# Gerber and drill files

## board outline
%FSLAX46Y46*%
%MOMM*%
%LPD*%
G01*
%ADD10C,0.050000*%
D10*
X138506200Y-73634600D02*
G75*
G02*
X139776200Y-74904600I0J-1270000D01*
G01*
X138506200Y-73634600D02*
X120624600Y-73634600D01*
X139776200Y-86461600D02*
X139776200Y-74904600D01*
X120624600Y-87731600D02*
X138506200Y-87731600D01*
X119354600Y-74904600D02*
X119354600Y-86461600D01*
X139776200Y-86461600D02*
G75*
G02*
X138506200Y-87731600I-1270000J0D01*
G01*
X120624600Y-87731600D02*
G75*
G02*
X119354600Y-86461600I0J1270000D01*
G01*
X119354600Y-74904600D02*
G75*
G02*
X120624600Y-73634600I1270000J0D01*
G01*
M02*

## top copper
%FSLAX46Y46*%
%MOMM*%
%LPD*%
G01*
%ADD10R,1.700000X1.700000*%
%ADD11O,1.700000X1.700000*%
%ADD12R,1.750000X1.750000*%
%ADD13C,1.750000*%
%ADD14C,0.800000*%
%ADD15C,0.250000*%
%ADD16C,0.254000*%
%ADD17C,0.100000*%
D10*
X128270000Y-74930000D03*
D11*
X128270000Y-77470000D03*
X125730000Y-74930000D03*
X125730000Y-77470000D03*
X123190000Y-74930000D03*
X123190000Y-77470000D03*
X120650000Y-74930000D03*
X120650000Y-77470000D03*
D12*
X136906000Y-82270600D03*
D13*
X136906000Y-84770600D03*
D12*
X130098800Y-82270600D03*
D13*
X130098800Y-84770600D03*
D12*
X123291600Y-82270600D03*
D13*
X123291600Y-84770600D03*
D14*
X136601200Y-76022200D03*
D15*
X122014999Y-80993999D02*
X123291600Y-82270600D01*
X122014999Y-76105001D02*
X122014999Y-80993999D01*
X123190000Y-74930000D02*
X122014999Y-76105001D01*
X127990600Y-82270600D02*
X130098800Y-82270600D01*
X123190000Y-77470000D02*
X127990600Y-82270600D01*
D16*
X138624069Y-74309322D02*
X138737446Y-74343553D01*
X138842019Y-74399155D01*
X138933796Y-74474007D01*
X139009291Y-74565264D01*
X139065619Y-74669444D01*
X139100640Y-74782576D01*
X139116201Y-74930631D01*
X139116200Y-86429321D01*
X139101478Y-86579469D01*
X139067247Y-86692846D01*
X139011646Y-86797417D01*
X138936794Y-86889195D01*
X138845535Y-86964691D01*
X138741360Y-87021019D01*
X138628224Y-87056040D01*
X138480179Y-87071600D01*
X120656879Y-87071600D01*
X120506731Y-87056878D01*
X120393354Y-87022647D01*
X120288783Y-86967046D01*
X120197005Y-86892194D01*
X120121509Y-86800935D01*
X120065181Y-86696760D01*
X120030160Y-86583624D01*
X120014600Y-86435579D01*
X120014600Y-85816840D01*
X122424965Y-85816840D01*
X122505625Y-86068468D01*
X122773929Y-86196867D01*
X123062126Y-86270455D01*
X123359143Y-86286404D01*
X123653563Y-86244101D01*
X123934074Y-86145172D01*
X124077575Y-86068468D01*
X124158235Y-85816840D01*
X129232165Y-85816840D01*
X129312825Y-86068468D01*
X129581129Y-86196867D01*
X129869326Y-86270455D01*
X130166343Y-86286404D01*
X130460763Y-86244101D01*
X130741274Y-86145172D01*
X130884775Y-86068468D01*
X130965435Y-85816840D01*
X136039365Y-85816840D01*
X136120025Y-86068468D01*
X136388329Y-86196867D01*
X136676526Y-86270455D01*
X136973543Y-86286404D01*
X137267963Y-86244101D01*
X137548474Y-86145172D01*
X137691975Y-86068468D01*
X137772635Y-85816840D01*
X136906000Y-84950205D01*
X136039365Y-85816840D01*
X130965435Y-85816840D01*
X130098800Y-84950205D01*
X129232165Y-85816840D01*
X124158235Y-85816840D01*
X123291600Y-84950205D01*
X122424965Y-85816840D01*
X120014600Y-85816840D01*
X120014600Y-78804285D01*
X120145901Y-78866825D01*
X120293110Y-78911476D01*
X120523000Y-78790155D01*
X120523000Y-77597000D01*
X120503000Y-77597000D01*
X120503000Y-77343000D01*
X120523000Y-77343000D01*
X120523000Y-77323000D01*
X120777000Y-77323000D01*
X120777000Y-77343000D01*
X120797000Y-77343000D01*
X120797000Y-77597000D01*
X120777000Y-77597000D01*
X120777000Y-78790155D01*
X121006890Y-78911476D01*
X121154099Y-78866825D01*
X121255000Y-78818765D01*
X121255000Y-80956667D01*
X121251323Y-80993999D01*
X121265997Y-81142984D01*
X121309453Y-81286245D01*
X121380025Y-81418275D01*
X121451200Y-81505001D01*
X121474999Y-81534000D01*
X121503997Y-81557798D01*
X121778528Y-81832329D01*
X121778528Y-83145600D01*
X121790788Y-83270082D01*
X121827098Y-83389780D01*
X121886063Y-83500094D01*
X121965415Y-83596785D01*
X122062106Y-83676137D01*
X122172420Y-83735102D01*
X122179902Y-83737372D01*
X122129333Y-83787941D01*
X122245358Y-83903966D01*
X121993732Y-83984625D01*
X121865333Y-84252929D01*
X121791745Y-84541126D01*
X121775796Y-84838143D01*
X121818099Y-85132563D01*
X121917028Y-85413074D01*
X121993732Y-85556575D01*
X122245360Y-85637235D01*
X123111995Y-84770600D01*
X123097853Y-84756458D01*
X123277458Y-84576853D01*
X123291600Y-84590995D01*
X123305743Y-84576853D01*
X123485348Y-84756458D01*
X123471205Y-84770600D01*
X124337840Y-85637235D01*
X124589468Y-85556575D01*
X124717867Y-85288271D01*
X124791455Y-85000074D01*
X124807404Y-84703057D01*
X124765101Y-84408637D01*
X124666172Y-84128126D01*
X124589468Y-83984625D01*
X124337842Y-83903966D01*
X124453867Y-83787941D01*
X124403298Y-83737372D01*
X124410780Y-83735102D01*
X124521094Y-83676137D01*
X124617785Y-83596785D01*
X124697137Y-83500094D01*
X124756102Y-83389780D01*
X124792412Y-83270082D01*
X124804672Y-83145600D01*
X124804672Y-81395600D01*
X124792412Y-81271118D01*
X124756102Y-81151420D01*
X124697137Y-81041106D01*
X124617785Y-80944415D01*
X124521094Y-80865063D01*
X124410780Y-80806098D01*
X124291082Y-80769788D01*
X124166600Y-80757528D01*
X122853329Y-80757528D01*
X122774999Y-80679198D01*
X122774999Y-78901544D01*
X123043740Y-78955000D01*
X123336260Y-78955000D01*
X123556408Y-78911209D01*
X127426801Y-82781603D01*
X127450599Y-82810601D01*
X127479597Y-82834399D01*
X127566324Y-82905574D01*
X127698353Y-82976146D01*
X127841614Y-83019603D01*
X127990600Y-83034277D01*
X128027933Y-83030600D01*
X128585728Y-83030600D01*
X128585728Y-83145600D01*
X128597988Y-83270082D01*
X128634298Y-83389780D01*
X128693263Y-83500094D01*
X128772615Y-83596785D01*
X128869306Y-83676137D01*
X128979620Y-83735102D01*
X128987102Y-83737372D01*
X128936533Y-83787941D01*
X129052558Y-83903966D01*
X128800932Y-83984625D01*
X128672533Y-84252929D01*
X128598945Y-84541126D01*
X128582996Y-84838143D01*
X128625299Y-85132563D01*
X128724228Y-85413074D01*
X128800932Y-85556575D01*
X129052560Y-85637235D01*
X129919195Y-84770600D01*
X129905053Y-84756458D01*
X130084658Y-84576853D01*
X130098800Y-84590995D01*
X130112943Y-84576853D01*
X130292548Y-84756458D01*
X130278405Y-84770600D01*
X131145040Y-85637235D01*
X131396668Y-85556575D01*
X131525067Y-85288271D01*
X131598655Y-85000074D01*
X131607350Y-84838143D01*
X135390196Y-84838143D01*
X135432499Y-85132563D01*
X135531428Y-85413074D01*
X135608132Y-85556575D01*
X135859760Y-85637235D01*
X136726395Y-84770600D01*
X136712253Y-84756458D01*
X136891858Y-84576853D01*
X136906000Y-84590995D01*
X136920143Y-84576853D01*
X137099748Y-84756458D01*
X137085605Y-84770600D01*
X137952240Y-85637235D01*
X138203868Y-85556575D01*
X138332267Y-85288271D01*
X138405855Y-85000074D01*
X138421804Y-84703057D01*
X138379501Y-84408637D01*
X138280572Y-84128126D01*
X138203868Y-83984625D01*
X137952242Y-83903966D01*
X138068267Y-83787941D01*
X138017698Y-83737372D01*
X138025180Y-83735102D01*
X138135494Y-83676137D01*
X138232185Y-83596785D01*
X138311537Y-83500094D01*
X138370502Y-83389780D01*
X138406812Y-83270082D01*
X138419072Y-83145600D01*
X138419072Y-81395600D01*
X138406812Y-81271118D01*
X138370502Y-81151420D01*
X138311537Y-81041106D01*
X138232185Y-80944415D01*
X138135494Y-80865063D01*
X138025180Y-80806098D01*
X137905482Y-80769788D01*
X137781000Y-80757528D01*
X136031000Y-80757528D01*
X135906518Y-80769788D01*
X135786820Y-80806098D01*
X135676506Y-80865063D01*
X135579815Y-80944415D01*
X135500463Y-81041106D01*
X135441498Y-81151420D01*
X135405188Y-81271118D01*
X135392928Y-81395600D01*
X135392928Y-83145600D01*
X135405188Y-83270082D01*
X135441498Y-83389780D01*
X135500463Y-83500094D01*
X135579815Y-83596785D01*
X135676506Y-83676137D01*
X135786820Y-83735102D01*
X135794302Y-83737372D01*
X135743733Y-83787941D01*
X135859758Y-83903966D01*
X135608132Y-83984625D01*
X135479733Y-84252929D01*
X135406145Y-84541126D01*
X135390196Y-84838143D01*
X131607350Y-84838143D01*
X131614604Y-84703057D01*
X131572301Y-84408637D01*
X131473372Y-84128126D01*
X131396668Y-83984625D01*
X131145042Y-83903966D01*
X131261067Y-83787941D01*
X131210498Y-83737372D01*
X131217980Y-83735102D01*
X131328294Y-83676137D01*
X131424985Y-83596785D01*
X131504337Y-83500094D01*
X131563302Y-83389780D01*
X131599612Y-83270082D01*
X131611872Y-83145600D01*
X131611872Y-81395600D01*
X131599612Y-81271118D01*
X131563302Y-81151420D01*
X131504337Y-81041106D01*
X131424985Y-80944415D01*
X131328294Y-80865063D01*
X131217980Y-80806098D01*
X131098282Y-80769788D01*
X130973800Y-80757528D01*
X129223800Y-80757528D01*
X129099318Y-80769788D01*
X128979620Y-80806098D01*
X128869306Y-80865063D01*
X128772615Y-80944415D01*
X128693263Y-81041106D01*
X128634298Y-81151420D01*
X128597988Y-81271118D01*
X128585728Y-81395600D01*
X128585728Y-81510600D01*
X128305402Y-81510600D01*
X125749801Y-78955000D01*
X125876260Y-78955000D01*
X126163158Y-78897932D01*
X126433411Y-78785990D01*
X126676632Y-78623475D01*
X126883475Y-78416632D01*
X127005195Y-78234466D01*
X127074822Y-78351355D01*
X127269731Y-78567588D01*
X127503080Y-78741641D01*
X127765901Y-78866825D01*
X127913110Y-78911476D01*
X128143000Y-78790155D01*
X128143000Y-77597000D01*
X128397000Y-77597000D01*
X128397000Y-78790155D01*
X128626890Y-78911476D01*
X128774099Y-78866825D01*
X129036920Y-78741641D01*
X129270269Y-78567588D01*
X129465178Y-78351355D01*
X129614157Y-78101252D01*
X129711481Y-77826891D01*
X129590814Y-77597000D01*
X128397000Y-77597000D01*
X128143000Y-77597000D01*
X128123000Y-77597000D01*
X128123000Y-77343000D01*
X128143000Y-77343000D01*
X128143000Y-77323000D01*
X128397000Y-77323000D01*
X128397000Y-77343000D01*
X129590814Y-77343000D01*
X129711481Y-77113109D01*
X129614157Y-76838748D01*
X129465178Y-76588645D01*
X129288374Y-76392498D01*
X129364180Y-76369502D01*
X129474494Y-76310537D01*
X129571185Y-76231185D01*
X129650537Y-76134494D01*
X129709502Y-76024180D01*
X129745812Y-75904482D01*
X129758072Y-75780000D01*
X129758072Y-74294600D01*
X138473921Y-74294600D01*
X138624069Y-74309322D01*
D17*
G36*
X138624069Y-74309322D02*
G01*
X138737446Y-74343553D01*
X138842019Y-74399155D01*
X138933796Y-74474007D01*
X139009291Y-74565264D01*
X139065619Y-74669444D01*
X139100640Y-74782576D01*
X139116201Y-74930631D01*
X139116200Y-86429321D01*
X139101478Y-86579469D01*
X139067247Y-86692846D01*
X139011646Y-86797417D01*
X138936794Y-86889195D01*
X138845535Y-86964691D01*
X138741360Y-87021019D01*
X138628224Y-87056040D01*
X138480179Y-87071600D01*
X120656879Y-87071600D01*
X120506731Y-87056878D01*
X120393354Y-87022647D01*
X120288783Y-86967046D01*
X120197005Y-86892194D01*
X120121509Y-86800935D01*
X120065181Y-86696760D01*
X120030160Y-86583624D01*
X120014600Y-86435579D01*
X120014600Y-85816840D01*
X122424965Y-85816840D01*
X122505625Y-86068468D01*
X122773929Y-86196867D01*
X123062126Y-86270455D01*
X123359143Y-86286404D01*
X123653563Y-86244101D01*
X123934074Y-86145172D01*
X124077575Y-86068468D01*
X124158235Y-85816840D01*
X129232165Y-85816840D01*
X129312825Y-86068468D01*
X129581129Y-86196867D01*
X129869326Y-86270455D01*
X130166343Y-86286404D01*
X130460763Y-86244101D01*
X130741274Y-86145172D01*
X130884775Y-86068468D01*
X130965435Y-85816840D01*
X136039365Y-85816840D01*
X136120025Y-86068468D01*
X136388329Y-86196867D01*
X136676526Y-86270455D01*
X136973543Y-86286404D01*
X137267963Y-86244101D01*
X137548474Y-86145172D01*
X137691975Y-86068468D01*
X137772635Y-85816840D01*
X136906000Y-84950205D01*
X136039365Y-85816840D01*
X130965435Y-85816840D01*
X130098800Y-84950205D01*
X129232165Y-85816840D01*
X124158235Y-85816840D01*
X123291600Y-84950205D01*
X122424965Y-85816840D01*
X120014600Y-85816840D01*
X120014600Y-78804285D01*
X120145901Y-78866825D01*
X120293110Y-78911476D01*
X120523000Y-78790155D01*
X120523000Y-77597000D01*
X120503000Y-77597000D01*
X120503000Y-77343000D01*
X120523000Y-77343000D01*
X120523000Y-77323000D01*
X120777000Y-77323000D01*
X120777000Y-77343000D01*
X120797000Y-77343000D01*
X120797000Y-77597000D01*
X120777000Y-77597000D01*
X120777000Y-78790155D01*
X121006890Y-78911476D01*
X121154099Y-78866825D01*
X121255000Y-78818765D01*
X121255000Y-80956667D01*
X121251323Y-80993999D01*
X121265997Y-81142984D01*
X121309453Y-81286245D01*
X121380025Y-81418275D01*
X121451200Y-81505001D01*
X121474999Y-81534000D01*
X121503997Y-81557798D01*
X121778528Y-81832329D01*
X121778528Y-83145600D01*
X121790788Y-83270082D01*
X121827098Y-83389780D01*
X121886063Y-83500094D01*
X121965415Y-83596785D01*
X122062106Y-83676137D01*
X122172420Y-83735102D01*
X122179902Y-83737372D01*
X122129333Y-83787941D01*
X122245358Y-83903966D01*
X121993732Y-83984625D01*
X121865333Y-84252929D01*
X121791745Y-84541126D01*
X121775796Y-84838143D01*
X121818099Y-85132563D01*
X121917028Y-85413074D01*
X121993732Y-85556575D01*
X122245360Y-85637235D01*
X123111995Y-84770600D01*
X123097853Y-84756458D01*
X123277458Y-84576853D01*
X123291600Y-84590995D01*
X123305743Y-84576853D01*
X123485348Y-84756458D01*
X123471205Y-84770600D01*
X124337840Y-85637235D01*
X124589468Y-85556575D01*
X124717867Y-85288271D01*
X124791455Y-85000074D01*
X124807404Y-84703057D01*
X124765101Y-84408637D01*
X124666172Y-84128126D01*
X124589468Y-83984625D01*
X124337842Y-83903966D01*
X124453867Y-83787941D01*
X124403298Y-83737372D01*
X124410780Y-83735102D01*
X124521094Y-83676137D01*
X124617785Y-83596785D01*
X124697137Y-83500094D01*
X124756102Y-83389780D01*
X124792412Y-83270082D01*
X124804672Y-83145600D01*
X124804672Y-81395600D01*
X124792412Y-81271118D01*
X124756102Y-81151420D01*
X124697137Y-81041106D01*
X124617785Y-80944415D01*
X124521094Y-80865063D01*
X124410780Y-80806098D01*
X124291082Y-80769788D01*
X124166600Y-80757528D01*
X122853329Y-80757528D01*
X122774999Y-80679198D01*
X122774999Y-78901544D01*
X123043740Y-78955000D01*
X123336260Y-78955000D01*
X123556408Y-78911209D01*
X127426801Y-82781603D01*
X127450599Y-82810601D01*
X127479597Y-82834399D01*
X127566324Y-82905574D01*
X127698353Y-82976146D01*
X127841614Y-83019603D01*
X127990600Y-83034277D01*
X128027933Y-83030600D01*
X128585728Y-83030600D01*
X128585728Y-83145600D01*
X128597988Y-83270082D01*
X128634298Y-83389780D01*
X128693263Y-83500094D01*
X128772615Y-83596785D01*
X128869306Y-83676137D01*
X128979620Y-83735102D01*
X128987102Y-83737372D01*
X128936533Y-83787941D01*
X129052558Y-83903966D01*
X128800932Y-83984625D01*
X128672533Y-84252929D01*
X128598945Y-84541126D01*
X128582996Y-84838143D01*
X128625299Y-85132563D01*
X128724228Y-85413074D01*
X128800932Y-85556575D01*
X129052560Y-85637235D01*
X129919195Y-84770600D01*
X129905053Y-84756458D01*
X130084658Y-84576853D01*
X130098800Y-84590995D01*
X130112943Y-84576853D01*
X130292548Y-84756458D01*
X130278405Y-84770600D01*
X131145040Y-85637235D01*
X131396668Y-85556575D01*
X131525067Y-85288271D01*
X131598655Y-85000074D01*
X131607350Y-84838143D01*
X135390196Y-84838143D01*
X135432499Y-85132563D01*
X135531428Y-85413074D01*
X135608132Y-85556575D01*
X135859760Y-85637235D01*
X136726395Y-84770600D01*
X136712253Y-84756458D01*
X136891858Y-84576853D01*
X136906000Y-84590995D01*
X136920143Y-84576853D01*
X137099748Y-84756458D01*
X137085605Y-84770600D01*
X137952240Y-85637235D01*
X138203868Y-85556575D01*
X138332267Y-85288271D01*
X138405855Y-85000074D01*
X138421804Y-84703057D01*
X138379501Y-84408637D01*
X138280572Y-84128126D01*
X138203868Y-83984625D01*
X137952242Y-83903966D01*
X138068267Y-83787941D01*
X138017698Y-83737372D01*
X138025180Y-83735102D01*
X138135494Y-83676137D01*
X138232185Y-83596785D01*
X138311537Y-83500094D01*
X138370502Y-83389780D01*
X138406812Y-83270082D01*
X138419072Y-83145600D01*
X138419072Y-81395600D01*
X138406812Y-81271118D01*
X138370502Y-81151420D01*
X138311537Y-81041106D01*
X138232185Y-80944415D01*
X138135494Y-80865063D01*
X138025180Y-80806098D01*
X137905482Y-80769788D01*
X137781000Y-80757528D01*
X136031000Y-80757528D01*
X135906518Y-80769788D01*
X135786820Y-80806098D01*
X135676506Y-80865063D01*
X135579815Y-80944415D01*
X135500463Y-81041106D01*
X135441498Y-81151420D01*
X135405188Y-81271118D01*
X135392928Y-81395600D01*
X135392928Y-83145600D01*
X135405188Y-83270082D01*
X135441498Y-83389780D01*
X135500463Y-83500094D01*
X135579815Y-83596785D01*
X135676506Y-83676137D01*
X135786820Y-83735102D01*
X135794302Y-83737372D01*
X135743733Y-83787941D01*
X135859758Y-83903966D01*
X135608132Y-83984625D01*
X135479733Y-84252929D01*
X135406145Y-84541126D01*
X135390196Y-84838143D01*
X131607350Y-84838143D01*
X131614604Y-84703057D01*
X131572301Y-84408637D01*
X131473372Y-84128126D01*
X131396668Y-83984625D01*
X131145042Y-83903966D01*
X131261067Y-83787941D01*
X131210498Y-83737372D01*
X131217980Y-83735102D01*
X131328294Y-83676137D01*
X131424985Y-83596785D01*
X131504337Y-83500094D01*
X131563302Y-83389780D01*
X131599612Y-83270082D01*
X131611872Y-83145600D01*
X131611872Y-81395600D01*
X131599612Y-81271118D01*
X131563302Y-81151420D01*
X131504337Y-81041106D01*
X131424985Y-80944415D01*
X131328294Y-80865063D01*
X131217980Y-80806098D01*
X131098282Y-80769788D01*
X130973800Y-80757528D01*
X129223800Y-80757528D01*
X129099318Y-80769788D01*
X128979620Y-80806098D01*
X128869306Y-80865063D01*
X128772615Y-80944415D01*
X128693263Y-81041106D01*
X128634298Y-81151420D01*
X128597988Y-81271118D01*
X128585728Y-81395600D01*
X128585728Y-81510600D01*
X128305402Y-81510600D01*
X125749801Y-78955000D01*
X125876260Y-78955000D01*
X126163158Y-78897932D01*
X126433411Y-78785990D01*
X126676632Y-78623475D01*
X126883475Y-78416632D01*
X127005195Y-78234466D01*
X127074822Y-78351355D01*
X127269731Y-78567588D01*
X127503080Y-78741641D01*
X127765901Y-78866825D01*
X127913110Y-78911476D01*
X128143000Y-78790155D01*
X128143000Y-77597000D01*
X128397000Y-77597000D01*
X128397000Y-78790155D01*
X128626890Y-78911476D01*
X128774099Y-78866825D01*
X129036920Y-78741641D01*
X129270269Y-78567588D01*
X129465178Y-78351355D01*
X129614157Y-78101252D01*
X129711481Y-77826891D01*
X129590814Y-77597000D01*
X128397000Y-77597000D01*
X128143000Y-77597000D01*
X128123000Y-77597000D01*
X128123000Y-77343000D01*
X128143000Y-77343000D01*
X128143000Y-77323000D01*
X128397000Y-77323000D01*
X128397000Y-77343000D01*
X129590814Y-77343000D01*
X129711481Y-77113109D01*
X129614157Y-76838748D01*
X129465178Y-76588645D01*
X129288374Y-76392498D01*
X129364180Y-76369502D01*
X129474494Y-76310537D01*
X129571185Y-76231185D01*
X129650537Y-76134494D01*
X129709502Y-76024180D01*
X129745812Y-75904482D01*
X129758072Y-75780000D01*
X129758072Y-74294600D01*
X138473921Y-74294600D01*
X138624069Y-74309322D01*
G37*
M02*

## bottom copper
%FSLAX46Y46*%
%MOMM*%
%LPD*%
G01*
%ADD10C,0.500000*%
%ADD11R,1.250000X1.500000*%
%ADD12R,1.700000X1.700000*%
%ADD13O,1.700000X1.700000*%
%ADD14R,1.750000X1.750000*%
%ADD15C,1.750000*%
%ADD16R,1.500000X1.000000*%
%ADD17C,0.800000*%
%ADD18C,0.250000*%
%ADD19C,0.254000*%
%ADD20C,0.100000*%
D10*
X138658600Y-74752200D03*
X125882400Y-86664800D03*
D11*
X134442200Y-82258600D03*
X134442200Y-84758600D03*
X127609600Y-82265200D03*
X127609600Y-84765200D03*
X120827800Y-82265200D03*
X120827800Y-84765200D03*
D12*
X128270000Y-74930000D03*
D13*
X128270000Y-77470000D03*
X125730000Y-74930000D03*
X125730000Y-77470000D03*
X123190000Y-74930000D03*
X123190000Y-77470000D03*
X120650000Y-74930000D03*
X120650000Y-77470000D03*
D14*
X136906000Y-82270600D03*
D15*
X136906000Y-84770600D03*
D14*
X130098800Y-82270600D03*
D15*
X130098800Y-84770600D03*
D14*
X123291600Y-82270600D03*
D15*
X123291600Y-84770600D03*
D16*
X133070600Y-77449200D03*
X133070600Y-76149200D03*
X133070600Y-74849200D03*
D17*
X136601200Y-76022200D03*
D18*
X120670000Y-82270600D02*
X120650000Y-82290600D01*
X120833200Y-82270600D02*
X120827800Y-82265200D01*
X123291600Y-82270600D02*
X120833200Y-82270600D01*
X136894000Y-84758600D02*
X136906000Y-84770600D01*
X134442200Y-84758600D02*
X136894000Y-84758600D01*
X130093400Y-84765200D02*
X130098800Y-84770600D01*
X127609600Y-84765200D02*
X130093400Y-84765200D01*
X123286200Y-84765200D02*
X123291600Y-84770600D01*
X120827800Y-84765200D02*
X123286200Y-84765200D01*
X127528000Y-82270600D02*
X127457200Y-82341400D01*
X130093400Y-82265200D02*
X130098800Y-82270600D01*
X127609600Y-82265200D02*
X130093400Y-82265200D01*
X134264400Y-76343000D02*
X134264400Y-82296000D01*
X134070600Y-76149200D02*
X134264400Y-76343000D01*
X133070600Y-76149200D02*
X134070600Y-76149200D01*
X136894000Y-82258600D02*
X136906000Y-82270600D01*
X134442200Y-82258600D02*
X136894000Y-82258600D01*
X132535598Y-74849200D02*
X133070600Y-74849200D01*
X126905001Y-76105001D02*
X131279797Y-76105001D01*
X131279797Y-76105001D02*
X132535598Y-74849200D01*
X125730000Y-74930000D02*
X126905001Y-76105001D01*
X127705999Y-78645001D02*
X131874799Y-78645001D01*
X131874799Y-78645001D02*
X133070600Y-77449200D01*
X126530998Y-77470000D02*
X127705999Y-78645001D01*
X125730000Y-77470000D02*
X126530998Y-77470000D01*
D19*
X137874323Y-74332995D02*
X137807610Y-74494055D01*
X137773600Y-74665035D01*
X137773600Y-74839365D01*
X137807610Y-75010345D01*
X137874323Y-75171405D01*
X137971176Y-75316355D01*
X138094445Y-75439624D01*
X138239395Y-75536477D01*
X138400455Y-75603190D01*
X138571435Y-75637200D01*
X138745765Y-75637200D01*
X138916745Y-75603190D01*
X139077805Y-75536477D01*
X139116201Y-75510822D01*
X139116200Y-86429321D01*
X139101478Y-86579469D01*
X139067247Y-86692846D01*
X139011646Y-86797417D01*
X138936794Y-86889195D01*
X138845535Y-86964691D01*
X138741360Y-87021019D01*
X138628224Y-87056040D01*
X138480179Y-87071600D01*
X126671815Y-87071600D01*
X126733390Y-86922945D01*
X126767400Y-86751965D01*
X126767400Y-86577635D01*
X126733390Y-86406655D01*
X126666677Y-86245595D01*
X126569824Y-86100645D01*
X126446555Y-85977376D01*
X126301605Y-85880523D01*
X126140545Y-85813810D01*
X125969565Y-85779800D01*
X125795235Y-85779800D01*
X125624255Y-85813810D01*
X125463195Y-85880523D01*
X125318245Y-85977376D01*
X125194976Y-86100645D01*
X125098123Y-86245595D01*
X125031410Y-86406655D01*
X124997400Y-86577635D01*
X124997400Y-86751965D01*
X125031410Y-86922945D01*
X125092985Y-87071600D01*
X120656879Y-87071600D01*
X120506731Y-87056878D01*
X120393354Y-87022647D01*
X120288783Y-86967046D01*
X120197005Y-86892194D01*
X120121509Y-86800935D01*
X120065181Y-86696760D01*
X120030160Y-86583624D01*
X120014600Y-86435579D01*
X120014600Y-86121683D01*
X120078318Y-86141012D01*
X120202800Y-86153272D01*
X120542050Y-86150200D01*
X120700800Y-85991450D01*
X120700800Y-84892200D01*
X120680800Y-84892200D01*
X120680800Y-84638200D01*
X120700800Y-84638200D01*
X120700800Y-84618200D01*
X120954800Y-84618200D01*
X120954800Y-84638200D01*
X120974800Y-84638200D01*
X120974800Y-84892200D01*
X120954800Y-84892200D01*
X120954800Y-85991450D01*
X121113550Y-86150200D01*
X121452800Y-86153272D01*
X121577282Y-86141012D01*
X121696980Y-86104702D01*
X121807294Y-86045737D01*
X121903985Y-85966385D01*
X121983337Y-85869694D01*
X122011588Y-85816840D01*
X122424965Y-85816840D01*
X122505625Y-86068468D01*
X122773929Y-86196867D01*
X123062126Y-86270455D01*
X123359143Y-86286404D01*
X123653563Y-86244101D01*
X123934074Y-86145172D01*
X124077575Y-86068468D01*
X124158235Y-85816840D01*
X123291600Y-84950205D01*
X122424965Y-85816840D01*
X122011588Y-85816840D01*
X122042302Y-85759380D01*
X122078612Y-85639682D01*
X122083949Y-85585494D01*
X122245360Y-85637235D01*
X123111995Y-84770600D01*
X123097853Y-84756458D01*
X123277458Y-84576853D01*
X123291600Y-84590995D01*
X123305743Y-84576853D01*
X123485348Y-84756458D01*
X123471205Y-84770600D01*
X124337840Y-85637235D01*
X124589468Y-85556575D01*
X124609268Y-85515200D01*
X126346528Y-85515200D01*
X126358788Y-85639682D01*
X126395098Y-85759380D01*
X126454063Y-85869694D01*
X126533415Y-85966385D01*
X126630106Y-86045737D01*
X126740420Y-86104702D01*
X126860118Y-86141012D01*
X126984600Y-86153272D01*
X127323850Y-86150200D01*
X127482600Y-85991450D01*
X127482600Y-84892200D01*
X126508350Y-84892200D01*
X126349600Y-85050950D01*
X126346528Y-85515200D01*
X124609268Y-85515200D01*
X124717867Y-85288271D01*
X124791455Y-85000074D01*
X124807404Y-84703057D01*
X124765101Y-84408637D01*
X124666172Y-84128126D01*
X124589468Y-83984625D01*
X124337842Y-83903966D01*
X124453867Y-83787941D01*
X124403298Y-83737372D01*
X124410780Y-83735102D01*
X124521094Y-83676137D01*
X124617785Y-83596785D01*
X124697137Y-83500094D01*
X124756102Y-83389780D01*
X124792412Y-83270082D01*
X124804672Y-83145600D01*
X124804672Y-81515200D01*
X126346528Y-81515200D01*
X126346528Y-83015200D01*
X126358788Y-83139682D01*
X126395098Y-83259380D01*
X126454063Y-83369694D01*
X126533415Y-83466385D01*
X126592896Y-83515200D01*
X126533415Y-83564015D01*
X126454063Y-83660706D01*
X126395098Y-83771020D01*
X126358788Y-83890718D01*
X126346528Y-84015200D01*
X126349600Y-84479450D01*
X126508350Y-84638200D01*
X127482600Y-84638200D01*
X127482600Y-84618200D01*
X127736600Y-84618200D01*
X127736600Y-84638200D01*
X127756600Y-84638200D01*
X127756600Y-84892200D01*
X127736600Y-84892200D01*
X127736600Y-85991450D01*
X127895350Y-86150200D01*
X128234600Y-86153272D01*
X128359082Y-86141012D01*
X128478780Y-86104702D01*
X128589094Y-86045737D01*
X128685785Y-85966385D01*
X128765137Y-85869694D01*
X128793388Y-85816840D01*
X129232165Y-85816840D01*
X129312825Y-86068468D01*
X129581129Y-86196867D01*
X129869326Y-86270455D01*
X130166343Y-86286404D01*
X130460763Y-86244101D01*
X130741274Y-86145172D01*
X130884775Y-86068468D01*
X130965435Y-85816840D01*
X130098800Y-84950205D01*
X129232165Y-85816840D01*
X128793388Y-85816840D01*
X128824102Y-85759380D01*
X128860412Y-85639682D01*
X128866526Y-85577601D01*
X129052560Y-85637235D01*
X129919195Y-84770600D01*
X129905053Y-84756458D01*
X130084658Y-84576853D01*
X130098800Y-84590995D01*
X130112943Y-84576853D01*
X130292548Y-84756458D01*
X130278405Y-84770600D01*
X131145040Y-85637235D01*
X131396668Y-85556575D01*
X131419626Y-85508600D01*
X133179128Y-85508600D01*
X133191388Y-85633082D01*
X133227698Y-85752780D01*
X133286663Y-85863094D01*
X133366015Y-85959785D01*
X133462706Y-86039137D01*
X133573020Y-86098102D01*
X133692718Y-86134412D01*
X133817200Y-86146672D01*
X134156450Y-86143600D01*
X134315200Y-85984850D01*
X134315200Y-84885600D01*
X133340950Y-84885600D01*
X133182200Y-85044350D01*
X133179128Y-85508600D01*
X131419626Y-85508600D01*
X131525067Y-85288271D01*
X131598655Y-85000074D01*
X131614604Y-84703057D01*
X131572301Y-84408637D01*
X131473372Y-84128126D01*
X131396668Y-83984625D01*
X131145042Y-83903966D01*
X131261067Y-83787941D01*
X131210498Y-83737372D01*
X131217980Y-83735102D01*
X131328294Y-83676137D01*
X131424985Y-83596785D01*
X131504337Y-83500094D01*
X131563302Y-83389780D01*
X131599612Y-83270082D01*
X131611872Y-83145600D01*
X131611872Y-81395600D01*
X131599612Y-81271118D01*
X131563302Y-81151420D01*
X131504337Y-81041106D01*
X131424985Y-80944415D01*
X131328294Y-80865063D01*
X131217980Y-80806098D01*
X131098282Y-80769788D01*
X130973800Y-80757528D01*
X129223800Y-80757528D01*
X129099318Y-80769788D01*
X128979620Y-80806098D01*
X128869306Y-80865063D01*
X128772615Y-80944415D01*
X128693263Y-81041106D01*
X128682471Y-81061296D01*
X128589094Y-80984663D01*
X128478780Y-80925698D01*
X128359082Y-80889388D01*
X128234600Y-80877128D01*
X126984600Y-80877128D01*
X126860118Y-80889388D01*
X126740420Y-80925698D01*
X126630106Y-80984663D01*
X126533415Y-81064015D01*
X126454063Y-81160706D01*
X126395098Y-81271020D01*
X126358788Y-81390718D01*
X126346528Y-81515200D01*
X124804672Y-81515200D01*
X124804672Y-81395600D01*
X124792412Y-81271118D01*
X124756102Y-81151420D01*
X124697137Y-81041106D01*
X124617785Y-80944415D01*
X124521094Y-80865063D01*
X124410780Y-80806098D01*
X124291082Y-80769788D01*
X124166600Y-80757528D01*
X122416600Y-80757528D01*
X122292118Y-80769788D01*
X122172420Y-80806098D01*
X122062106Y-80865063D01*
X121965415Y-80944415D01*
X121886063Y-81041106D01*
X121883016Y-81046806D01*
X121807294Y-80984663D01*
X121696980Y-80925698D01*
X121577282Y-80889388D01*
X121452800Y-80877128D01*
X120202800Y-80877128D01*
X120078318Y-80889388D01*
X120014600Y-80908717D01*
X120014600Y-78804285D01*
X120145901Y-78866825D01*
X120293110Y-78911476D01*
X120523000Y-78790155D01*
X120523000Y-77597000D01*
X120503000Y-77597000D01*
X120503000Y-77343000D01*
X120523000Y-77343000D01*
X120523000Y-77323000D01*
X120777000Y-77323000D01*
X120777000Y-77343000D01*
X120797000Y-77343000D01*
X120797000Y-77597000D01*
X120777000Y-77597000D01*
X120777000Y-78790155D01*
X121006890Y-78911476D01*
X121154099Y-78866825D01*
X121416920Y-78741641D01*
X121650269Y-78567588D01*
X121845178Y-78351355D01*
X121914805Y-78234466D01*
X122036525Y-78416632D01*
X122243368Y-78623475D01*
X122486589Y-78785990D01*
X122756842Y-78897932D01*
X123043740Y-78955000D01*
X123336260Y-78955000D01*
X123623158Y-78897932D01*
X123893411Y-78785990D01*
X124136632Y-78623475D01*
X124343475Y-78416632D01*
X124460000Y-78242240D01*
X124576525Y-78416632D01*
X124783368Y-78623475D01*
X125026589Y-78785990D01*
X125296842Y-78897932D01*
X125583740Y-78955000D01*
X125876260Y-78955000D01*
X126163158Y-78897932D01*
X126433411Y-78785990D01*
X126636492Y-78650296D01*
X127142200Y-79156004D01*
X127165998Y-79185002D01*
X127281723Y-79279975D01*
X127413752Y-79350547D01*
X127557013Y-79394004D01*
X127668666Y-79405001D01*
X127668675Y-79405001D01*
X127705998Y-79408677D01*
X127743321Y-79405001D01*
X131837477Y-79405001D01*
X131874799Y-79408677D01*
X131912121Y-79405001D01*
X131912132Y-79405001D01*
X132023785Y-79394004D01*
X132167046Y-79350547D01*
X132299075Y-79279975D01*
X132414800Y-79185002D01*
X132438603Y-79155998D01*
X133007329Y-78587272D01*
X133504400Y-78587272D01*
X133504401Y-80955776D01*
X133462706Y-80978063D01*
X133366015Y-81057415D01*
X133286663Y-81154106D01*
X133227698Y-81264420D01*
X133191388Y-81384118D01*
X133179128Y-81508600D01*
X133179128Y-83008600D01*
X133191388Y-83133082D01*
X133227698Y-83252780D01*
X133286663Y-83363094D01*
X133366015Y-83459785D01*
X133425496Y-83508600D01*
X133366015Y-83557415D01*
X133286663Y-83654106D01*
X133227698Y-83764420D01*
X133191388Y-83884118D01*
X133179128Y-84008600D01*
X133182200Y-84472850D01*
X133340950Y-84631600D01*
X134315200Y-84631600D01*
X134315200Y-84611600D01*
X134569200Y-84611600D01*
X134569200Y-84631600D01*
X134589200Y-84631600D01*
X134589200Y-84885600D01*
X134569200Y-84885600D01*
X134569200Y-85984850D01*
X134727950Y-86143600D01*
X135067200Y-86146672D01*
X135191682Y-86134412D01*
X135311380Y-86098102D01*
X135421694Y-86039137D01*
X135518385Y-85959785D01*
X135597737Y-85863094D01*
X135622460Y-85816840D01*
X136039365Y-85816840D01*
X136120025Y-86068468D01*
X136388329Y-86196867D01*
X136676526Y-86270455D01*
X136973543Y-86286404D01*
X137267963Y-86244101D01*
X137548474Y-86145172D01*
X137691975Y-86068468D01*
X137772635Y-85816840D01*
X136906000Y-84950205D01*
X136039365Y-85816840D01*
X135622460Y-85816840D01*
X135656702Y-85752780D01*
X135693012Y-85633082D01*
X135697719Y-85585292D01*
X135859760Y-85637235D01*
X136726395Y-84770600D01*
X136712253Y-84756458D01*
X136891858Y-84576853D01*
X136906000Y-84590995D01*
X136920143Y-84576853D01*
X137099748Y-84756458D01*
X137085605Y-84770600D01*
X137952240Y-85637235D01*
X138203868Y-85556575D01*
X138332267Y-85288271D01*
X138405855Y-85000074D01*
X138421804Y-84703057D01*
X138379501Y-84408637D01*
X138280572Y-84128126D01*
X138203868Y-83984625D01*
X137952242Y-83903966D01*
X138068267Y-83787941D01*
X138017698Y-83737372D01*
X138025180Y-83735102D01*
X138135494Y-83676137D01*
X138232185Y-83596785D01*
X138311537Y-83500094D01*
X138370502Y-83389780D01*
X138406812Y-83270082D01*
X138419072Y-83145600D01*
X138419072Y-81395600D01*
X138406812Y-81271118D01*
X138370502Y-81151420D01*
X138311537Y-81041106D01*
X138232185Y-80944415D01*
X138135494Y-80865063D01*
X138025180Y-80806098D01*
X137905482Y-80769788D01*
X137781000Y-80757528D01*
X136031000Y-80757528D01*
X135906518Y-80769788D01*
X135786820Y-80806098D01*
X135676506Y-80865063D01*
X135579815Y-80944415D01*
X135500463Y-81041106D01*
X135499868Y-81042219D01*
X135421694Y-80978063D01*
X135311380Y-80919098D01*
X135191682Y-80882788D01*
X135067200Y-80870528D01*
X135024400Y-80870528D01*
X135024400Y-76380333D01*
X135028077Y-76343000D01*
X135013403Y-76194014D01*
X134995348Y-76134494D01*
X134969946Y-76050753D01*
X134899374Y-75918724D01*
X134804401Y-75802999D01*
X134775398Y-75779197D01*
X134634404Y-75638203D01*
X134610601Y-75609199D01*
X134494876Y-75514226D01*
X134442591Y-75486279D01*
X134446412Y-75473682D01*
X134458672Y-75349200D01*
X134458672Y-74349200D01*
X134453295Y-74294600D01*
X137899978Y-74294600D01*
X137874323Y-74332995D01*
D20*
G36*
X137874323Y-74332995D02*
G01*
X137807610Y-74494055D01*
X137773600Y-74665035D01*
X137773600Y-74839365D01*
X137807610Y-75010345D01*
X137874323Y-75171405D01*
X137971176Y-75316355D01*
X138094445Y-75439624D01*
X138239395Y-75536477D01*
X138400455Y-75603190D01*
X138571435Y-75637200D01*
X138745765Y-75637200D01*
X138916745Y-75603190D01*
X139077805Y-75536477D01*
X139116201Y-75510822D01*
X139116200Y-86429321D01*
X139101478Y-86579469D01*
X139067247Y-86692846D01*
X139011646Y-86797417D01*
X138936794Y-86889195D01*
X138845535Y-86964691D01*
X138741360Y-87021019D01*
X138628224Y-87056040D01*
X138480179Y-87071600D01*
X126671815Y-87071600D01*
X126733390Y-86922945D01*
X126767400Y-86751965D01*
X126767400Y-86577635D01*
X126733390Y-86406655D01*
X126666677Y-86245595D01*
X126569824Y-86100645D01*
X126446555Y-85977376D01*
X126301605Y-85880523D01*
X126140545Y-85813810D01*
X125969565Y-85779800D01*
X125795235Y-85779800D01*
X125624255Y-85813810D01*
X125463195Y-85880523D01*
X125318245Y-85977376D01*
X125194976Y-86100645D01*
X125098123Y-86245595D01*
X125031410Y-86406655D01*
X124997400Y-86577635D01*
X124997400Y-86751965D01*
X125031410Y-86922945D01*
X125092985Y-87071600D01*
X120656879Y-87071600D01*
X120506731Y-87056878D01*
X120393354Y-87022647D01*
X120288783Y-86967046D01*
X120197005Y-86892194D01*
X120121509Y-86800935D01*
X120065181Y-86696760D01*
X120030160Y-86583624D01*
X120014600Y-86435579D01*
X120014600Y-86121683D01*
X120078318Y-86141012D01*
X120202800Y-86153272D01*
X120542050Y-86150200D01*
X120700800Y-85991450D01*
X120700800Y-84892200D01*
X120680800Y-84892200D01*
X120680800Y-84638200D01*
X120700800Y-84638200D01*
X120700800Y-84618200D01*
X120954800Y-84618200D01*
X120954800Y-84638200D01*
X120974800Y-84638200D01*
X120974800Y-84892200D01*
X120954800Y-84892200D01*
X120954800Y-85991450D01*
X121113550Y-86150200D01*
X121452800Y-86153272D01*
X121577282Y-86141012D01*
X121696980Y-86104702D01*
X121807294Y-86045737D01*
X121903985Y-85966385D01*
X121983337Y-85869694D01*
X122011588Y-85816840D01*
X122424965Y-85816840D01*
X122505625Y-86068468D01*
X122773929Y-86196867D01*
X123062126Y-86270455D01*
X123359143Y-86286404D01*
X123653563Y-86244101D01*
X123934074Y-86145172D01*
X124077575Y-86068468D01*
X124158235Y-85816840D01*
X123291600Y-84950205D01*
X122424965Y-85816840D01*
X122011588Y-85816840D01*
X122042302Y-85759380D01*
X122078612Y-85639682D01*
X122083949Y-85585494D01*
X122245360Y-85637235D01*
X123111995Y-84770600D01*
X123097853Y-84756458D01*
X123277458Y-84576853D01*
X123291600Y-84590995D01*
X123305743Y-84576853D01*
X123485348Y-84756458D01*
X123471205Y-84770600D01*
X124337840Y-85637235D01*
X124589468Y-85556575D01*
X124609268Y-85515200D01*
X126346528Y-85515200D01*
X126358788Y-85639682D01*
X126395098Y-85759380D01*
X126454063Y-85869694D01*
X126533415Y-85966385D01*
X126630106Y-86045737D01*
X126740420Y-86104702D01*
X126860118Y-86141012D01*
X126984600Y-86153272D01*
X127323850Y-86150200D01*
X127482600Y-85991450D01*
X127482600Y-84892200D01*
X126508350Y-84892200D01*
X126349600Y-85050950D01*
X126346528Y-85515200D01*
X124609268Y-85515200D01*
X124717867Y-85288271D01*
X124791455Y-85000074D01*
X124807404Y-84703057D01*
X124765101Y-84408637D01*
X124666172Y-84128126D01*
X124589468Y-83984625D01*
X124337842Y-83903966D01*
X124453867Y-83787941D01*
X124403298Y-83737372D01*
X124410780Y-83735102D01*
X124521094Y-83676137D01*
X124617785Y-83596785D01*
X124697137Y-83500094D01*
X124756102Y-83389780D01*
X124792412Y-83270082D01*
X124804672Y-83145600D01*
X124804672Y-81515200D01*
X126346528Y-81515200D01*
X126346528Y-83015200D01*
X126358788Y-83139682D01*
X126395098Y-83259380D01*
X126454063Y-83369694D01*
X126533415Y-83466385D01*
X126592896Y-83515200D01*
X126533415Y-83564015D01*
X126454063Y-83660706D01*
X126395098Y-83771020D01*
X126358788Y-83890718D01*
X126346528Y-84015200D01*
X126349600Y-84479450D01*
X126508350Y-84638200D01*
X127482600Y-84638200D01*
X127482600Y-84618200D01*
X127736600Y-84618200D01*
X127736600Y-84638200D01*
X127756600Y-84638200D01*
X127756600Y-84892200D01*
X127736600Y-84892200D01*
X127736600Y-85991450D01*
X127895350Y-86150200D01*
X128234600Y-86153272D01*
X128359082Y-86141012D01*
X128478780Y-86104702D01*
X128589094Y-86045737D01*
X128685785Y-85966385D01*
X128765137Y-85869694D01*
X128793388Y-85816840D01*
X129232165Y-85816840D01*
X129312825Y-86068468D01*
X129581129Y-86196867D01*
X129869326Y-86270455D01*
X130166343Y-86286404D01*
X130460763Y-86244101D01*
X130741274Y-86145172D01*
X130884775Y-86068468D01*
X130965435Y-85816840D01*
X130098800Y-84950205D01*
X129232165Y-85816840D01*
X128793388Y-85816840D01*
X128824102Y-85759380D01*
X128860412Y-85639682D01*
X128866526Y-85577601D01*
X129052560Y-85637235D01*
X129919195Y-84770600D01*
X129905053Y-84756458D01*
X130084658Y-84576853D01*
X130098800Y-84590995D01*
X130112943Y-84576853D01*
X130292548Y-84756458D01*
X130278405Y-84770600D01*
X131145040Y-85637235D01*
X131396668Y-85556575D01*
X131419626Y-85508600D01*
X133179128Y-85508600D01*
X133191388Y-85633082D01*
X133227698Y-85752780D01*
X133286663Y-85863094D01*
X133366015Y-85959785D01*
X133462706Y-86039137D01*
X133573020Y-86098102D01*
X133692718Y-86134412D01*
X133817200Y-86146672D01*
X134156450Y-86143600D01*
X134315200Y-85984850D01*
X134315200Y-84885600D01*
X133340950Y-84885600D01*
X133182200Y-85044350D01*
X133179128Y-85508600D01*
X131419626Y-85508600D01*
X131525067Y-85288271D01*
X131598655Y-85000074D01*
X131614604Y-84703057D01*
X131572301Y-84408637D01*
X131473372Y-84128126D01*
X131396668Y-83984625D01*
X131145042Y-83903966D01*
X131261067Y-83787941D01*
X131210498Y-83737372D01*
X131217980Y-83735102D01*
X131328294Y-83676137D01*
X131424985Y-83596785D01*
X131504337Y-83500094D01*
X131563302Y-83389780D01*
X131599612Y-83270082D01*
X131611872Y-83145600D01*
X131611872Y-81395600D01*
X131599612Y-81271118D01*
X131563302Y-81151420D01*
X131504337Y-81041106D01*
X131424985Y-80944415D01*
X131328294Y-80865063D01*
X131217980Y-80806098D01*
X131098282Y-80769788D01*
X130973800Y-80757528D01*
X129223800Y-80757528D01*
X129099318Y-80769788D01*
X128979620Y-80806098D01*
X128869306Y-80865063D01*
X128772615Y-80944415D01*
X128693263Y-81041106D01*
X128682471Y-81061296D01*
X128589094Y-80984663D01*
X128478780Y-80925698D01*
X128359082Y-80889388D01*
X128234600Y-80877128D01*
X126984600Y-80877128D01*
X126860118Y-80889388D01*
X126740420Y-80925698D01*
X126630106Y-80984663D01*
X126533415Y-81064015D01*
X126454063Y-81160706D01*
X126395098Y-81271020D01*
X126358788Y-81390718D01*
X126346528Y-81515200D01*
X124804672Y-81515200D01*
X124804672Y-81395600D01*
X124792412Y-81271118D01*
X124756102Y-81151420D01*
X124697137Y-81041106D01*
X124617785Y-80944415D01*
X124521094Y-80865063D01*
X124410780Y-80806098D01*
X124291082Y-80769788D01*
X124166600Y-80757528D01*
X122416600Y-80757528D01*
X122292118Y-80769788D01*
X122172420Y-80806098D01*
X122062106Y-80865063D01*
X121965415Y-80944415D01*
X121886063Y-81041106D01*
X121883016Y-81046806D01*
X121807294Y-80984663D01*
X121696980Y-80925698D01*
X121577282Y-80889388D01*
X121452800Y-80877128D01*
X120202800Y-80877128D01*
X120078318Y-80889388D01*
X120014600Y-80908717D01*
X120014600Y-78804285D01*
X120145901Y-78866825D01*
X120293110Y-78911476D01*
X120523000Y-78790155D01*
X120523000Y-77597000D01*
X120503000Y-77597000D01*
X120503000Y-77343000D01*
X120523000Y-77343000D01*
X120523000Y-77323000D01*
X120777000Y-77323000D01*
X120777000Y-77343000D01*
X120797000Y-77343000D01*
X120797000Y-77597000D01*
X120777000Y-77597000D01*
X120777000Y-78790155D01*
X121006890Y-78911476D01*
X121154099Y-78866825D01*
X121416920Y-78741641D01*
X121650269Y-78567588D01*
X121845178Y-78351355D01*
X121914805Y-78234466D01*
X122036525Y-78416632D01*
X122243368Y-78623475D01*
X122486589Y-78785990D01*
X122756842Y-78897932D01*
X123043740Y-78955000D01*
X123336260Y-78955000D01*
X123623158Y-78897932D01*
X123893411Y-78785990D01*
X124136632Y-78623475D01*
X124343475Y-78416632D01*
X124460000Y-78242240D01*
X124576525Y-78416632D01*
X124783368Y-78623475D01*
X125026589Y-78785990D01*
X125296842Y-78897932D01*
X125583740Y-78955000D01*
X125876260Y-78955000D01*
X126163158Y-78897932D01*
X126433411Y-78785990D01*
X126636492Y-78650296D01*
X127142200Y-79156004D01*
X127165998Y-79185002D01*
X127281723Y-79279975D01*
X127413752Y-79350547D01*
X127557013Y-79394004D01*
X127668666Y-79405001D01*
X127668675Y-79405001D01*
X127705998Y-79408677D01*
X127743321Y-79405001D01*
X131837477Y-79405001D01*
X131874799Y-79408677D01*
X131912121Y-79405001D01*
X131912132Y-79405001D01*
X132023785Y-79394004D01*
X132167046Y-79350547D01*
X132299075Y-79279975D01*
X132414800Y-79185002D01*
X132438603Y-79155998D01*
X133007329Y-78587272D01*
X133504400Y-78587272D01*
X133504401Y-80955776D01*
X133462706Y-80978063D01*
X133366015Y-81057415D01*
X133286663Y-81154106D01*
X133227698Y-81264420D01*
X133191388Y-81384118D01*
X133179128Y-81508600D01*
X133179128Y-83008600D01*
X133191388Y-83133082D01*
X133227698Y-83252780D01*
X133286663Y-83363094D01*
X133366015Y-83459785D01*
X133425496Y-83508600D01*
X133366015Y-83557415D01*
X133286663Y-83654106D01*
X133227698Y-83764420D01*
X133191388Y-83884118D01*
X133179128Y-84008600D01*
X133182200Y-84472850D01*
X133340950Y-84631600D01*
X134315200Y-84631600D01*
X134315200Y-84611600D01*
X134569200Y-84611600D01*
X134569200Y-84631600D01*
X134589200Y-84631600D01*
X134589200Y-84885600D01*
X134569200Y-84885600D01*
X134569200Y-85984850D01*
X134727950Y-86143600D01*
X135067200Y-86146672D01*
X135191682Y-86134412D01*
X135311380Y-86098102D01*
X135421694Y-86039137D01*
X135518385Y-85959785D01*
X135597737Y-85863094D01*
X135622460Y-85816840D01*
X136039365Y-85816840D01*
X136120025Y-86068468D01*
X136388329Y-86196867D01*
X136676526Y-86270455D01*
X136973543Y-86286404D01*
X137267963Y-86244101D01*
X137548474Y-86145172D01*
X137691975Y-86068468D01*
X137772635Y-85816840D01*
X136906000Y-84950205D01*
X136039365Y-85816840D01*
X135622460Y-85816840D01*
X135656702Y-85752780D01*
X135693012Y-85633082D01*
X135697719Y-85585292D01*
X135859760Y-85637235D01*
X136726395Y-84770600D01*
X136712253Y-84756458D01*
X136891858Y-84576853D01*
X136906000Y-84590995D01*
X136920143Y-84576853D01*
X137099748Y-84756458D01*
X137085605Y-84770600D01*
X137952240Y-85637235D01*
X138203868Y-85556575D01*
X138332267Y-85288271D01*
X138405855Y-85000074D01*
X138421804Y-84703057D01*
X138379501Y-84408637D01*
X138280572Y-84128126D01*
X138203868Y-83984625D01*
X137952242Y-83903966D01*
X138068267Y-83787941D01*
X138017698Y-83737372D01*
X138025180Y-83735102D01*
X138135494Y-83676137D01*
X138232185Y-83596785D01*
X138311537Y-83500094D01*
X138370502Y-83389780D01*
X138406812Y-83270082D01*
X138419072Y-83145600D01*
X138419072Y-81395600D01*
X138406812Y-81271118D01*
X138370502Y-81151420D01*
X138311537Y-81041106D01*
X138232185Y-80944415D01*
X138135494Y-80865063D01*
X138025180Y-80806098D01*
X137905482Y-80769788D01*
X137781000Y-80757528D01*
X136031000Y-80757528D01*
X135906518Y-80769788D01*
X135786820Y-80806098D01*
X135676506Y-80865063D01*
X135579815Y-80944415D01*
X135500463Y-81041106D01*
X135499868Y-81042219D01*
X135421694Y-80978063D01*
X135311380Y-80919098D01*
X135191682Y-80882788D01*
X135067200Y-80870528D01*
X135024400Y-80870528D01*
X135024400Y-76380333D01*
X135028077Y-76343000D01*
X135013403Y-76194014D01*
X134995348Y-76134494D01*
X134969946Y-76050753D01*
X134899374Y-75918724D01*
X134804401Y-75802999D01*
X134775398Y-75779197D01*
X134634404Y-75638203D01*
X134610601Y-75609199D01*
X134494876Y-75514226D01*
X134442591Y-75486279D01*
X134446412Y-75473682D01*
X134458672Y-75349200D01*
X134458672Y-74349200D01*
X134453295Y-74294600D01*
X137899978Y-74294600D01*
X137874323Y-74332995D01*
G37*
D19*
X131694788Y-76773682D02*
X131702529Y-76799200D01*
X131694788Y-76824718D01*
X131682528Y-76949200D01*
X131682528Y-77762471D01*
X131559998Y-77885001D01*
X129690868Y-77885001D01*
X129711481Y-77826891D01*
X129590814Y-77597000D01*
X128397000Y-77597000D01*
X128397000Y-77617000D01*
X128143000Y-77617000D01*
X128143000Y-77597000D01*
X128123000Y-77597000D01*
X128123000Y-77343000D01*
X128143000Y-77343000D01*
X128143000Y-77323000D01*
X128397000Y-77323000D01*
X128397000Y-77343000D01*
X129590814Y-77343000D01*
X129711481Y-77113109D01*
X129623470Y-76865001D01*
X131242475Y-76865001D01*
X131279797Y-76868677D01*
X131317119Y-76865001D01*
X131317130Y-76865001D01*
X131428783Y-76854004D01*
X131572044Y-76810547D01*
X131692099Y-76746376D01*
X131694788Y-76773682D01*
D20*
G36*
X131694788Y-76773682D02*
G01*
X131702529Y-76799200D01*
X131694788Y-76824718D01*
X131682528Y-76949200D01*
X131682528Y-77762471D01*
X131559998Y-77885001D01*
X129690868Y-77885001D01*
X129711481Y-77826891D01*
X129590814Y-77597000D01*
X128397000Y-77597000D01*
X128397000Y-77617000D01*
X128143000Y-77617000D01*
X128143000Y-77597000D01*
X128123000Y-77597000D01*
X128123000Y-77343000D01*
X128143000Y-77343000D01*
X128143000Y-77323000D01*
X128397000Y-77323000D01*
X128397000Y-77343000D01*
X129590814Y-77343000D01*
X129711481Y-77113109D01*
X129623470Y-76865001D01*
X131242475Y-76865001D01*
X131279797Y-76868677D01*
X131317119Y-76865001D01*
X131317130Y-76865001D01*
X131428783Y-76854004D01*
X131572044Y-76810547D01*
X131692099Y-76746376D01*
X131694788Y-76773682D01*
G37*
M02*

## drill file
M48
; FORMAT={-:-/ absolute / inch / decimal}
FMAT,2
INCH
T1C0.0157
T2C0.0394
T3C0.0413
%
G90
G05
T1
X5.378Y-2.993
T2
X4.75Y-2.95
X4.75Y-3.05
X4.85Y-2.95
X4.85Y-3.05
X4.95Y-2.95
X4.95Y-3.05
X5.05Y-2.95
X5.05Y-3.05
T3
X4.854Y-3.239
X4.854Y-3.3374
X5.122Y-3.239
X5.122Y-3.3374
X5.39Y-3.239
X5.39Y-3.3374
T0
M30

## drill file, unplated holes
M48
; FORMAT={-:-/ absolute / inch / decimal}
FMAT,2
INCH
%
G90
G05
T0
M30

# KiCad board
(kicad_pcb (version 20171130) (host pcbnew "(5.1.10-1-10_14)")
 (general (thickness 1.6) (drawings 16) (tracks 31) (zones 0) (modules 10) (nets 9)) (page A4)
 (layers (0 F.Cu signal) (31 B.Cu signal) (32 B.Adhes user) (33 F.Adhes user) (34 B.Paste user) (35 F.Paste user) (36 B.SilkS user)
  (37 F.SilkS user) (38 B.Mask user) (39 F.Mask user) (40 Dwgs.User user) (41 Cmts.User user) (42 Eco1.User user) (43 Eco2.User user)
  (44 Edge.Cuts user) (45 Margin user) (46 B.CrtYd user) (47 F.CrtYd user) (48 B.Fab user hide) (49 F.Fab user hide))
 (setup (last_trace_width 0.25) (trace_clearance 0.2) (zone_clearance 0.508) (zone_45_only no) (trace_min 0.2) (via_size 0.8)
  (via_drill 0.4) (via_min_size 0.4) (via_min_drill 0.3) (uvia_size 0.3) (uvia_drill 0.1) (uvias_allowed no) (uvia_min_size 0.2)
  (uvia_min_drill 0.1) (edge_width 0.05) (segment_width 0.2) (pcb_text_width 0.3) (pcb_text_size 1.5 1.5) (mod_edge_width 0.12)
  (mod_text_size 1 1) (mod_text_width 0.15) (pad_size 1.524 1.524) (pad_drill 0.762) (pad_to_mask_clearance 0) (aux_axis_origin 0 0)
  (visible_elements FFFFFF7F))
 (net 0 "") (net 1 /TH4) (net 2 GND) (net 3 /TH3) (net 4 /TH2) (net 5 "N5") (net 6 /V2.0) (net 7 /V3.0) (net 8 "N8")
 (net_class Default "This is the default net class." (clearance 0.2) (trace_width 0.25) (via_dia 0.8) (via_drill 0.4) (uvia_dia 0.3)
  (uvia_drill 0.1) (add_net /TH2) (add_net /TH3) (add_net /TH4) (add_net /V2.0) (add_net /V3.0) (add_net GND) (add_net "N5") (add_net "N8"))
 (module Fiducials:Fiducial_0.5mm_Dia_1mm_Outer (layer B.Cu) (at 138.6586 74.7522)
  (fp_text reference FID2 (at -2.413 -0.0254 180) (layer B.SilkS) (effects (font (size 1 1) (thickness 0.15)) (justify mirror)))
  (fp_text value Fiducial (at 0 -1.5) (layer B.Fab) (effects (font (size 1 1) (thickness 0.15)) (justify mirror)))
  (pad ~ smd circle (at 0 0) (size 0.5 0.5) (layers B.Cu B.Mask) (solder_mask_margin 0.25) (clearance 0.25)))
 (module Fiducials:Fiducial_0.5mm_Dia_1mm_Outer (layer B.Cu) (at 125.8824 86.6648)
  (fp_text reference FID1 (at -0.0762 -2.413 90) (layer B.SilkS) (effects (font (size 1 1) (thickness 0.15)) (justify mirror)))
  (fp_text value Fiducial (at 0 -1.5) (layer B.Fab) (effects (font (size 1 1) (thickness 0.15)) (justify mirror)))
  (pad ~ smd circle (at 0 0) (size 0.5 0.5) (layers B.Cu B.Mask) (solder_mask_margin 0.25) (clearance 0.25)))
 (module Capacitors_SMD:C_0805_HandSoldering (layer B.Cu) (at 134.4422 83.5086 270)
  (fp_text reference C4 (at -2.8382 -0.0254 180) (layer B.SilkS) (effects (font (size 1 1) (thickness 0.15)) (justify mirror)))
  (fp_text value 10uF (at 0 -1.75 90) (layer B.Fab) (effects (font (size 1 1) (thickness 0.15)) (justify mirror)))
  (pad 1 smd rect (at -1.25 0 270) (size 1.5 1.25) (layers B.Cu B.Paste B.Mask) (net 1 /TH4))
  (pad 2 smd rect (at 1.25 0 270) (size 1.5 1.25) (layers B.Cu B.Paste B.Mask) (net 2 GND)))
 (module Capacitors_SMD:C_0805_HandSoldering (layer B.Cu) (at 127.6096 83.5152 270)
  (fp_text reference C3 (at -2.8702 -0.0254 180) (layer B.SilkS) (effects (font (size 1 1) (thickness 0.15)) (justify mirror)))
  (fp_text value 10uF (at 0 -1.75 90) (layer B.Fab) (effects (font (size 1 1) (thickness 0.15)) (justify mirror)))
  (pad 1 smd rect (at -1.25 0 270) (size 1.5 1.25) (layers B.Cu B.Paste B.Mask) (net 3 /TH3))
  (pad 2 smd rect (at 1.25 0 270) (size 1.5 1.25) (layers B.Cu B.Paste B.Mask) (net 2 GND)))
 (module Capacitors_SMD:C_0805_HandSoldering (layer B.Cu) (at 120.8278 83.5152 270)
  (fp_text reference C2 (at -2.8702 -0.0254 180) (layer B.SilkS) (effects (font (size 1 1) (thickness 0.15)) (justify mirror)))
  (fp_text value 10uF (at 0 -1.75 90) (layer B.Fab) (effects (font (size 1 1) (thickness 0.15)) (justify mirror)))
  (pad 1 smd rect (at -1.25 0 270) (size 1.5 1.25) (layers B.Cu B.Paste B.Mask) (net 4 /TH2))
  (pad 2 smd rect (at 1.25 0 270) (size 1.5 1.25) (layers B.Cu B.Paste B.Mask) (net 2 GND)))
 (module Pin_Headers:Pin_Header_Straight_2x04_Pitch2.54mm (layer F.Cu) (at 128.27 74.93 270)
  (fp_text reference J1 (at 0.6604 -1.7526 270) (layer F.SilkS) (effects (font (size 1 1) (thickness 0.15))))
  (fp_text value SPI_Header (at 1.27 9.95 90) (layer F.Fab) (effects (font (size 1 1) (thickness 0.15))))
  (pad 1 thru_hole rect (at 0 0 270) (size 1.7 1.7) (drill 1) (layers *.Cu *.Mask) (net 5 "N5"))
  (pad 2 thru_hole oval (at 2.54 0 270) (size 1.7 1.7) (drill 1) (layers *.Cu *.Mask) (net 2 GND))
  (pad 3 thru_hole oval (at 0 2.54 270) (size 1.7 1.7) (drill 1) (layers *.Cu *.Mask) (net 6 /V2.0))
  (pad 4 thru_hole oval (at 2.54 2.54 270) (size 1.7 1.7) (drill 1) (layers *.Cu *.Mask) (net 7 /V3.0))
  (pad 5 thru_hole oval (at 0 5.08 270) (size 1.7 1.7) (drill 1) (layers *.Cu *.Mask) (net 4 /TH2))
  (pad 6 thru_hole oval (at 2.54 5.08 270) (size 1.7 1.7) (drill 1) (layers *.Cu *.Mask) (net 3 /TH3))
  (pad 7 thru_hole oval (at 0 7.62 270) (size 1.7 1.7) (drill 1) (layers *.Cu *.Mask) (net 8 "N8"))
  (pad 8 thru_hole oval (at 2.54 7.62 270) (size 1.7 1.7) (drill 1) (layers *.Cu *.Mask) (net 2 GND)))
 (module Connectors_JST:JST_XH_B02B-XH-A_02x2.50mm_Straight (layer F.Cu) (at 136.906 82.2706 270)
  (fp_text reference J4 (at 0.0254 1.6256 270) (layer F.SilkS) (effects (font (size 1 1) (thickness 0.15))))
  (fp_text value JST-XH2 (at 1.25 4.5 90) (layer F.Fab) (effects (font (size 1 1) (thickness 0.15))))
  (pad 1 thru_hole rect (at 0 0 270) (size 1.75 1.75) (drill 1.05) (layers *.Cu *.Mask) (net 1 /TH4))
  (pad 2 thru_hole circle (at 2.5 0 270) (size 1.75 1.75) (drill 1.05) (layers *.Cu *.Mask) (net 2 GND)))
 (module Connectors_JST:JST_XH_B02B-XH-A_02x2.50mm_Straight (layer F.Cu) (at 130.0988 82.2706 270)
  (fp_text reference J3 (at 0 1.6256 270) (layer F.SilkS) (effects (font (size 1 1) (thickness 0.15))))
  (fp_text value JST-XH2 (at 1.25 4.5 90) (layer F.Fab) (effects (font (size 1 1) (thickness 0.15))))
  (pad 1 thru_hole rect (at 0 0 270) (size 1.75 1.75) (drill 1.05) (layers *.Cu *.Mask) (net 3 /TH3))
  (pad 2 thru_hole circle (at 2.5 0 270) (size 1.75 1.75) (drill 1.05) (layers *.Cu *.Mask) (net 2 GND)))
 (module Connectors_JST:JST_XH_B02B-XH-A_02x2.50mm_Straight (layer F.Cu) (at 123.2916 82.2706 270)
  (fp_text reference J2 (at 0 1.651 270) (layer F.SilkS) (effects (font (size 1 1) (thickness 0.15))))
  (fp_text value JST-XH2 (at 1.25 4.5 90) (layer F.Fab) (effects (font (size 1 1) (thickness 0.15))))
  (pad 1 thru_hole rect (at 0 0 270) (size 1.75 1.75) (drill 1.05) (layers *.Cu *.Mask) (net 4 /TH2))
  (pad 2 thru_hole circle (at 2.5 0 270) (size 1.75 1.75) (drill 1.05) (layers *.Cu *.Mask) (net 2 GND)))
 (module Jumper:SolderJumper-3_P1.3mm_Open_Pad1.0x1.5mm (layer B.Cu) (at 133.0706 76.1492 90)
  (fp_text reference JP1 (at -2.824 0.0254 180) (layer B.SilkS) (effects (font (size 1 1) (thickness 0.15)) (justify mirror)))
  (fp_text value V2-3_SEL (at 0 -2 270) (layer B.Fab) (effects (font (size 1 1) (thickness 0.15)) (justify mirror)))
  (pad 1 smd rect (at -1.3 0 90) (size 1 1.5) (layers B.Cu B.Mask) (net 7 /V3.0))
  (pad 2 smd rect (at 0 0 90) (size 1 1.5) (layers B.Cu B.Mask) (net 1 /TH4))
  (pad 3 smd rect (at 1.3 0 90) (size 1 1.5) (layers B.Cu B.Mask) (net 6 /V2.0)))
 (gr_arc (start 138.5062 74.9046) (end 139.7762 74.9046) (angle -90) (layer Edge.Cuts) (width 0.05))
 (gr_line (start 138.5062 73.6346) (end 120.6246 73.6346) (layer Edge.Cuts) (width 0.05))
 (gr_line (start 139.7762 86.4616) (end 139.7762 74.9046) (layer Edge.Cuts) (width 0.05))
 (gr_line (start 120.6246 87.7316) (end 138.5062 87.7316) (layer Edge.Cuts) (width 0.05))
 (gr_line (start 119.3546 74.9046) (end 119.3546 86.4616) (layer Edge.Cuts) (width 0.05))
 (gr_arc (start 138.5062 86.4616) (end 138.5062 87.7316) (angle -90) (layer Edge.Cuts) (width 0.05))
 (gr_arc (start 120.6246 86.4616) (end 119.3546 86.4616) (angle -90) (layer Edge.Cuts) (width 0.05))
 (gr_arc (start 120.6246 74.9046) (end 120.6246 73.6346) (angle -90) (layer Edge.Cuts) (width 0.05))
 (segment (start 122.014999 80.993999) (end 123.2916 82.2706) (width 0.25) (layer F.Cu) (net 4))
 (segment (start 122.014999 76.105001) (end 122.014999 80.993999) (width 0.25) (layer F.Cu) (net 4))
 (segment (start 123.19 74.93) (end 122.014999 76.105001) (width 0.25) (layer F.Cu) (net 4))
 (segment (start 120.67 82.2706) (end 120.65 82.2906) (width 0.25) (layer B.Cu) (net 4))
 (segment (start 120.8332 82.2706) (end 120.8278 82.2652) (width 0.25) (layer B.Cu) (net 4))
 (segment (start 123.2916 82.2706) (end 120.8332 82.2706) (width 0.25) (layer B.Cu) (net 4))
 (via (at 136.6012 76.0222) (size 0.8) (drill 0.4) (layers F.Cu B.Cu) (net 2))
 (segment (start 136.894 84.7586) (end 136.906 84.7706) (width 0.25) (layer B.Cu) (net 2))
 (segment (start 134.4422 84.7586) (end 136.894 84.7586) (width 0.25) (layer B.Cu) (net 2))
 (segment (start 130.0934 84.7652) (end 130.0988 84.7706) (width 0.25) (layer B.Cu) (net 2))
 (segment (start 127.6096 84.7652) (end 130.0934 84.7652) (width 0.25) (layer B.Cu) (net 2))
 (segment (start 123.2862 84.7652) (end 123.2916 84.7706) (width 0.25) (layer B.Cu) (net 2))
 (segment (start 120.8278 84.7652) (end 123.2862 84.7652) (width 0.25) (layer B.Cu) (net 2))
 (segment (start 127.9906 82.2706) (end 130.0988 82.2706) (width 0.25) (layer F.Cu) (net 3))
 (segment (start 123.19 77.47) (end 127.9906 82.2706) (width 0.25) (layer F.Cu) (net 3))
 (segment (start 127.528 82.2706) (end 127.4572 82.3414) (width 0.25) (layer B.Cu) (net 3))
 (segment (start 130.0934 82.2652) (end 130.0988 82.2706) (width 0.25) (layer B.Cu) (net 3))
 (segment (start 127.6096 82.2652) (end 130.0934 82.2652) (width 0.25) (layer B.Cu) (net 3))
 (segment (start 134.2644 76.343) (end 134.2644 82.296) (width 0.25) (layer B.Cu) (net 1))
 (segment (start 134.0706 76.1492) (end 134.2644 76.343) (width 0.25) (layer B.Cu) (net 1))
 (segment (start 133.0706 76.1492) (end 134.0706 76.1492) (width 0.25) (layer B.Cu) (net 1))
 (segment (start 136.894 82.2586) (end 136.906 82.2706) (width 0.25) (layer B.Cu) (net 1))
 (segment (start 134.4422 82.2586) (end 136.894 82.2586) (width 0.25) (layer B.Cu) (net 1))
 (segment (start 132.535598 74.8492) (end 133.0706 74.8492) (width 0.25) (layer B.Cu) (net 6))
 (segment (start 126.905001 76.105001) (end 131.279797 76.105001) (width 0.25) (layer B.Cu) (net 6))
 (segment (start 131.279797 76.105001) (end 132.535598 74.8492) (width 0.25) (layer B.Cu) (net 6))
 (segment (start 125.73 74.93) (end 126.905001 76.105001) (width 0.25) (layer B.Cu) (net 6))
 (segment (start 127.705999 78.645001) (end 131.874799 78.645001) (width 0.25) (layer B.Cu) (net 7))
 (segment (start 131.874799 78.645001) (end 133.0706 77.4492) (width 0.25) (layer B.Cu) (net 7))
 (segment (start 126.530998 77.47) (end 127.705999 78.645001) (width 0.25) (layer B.Cu) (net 7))
 (segment (start 125.73 77.47) (end 126.530998 77.47) (width 0.25) (layer B.Cu) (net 7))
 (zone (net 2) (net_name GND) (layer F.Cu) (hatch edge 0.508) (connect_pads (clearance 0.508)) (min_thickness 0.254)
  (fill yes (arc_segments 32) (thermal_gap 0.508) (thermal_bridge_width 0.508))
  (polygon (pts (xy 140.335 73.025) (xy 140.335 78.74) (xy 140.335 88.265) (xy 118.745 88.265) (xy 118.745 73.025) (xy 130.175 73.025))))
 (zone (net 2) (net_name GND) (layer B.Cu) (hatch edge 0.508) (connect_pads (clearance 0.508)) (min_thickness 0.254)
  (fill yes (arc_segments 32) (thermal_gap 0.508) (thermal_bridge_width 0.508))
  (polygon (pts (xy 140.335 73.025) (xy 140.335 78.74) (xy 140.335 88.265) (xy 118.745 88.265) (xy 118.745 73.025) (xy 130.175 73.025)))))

